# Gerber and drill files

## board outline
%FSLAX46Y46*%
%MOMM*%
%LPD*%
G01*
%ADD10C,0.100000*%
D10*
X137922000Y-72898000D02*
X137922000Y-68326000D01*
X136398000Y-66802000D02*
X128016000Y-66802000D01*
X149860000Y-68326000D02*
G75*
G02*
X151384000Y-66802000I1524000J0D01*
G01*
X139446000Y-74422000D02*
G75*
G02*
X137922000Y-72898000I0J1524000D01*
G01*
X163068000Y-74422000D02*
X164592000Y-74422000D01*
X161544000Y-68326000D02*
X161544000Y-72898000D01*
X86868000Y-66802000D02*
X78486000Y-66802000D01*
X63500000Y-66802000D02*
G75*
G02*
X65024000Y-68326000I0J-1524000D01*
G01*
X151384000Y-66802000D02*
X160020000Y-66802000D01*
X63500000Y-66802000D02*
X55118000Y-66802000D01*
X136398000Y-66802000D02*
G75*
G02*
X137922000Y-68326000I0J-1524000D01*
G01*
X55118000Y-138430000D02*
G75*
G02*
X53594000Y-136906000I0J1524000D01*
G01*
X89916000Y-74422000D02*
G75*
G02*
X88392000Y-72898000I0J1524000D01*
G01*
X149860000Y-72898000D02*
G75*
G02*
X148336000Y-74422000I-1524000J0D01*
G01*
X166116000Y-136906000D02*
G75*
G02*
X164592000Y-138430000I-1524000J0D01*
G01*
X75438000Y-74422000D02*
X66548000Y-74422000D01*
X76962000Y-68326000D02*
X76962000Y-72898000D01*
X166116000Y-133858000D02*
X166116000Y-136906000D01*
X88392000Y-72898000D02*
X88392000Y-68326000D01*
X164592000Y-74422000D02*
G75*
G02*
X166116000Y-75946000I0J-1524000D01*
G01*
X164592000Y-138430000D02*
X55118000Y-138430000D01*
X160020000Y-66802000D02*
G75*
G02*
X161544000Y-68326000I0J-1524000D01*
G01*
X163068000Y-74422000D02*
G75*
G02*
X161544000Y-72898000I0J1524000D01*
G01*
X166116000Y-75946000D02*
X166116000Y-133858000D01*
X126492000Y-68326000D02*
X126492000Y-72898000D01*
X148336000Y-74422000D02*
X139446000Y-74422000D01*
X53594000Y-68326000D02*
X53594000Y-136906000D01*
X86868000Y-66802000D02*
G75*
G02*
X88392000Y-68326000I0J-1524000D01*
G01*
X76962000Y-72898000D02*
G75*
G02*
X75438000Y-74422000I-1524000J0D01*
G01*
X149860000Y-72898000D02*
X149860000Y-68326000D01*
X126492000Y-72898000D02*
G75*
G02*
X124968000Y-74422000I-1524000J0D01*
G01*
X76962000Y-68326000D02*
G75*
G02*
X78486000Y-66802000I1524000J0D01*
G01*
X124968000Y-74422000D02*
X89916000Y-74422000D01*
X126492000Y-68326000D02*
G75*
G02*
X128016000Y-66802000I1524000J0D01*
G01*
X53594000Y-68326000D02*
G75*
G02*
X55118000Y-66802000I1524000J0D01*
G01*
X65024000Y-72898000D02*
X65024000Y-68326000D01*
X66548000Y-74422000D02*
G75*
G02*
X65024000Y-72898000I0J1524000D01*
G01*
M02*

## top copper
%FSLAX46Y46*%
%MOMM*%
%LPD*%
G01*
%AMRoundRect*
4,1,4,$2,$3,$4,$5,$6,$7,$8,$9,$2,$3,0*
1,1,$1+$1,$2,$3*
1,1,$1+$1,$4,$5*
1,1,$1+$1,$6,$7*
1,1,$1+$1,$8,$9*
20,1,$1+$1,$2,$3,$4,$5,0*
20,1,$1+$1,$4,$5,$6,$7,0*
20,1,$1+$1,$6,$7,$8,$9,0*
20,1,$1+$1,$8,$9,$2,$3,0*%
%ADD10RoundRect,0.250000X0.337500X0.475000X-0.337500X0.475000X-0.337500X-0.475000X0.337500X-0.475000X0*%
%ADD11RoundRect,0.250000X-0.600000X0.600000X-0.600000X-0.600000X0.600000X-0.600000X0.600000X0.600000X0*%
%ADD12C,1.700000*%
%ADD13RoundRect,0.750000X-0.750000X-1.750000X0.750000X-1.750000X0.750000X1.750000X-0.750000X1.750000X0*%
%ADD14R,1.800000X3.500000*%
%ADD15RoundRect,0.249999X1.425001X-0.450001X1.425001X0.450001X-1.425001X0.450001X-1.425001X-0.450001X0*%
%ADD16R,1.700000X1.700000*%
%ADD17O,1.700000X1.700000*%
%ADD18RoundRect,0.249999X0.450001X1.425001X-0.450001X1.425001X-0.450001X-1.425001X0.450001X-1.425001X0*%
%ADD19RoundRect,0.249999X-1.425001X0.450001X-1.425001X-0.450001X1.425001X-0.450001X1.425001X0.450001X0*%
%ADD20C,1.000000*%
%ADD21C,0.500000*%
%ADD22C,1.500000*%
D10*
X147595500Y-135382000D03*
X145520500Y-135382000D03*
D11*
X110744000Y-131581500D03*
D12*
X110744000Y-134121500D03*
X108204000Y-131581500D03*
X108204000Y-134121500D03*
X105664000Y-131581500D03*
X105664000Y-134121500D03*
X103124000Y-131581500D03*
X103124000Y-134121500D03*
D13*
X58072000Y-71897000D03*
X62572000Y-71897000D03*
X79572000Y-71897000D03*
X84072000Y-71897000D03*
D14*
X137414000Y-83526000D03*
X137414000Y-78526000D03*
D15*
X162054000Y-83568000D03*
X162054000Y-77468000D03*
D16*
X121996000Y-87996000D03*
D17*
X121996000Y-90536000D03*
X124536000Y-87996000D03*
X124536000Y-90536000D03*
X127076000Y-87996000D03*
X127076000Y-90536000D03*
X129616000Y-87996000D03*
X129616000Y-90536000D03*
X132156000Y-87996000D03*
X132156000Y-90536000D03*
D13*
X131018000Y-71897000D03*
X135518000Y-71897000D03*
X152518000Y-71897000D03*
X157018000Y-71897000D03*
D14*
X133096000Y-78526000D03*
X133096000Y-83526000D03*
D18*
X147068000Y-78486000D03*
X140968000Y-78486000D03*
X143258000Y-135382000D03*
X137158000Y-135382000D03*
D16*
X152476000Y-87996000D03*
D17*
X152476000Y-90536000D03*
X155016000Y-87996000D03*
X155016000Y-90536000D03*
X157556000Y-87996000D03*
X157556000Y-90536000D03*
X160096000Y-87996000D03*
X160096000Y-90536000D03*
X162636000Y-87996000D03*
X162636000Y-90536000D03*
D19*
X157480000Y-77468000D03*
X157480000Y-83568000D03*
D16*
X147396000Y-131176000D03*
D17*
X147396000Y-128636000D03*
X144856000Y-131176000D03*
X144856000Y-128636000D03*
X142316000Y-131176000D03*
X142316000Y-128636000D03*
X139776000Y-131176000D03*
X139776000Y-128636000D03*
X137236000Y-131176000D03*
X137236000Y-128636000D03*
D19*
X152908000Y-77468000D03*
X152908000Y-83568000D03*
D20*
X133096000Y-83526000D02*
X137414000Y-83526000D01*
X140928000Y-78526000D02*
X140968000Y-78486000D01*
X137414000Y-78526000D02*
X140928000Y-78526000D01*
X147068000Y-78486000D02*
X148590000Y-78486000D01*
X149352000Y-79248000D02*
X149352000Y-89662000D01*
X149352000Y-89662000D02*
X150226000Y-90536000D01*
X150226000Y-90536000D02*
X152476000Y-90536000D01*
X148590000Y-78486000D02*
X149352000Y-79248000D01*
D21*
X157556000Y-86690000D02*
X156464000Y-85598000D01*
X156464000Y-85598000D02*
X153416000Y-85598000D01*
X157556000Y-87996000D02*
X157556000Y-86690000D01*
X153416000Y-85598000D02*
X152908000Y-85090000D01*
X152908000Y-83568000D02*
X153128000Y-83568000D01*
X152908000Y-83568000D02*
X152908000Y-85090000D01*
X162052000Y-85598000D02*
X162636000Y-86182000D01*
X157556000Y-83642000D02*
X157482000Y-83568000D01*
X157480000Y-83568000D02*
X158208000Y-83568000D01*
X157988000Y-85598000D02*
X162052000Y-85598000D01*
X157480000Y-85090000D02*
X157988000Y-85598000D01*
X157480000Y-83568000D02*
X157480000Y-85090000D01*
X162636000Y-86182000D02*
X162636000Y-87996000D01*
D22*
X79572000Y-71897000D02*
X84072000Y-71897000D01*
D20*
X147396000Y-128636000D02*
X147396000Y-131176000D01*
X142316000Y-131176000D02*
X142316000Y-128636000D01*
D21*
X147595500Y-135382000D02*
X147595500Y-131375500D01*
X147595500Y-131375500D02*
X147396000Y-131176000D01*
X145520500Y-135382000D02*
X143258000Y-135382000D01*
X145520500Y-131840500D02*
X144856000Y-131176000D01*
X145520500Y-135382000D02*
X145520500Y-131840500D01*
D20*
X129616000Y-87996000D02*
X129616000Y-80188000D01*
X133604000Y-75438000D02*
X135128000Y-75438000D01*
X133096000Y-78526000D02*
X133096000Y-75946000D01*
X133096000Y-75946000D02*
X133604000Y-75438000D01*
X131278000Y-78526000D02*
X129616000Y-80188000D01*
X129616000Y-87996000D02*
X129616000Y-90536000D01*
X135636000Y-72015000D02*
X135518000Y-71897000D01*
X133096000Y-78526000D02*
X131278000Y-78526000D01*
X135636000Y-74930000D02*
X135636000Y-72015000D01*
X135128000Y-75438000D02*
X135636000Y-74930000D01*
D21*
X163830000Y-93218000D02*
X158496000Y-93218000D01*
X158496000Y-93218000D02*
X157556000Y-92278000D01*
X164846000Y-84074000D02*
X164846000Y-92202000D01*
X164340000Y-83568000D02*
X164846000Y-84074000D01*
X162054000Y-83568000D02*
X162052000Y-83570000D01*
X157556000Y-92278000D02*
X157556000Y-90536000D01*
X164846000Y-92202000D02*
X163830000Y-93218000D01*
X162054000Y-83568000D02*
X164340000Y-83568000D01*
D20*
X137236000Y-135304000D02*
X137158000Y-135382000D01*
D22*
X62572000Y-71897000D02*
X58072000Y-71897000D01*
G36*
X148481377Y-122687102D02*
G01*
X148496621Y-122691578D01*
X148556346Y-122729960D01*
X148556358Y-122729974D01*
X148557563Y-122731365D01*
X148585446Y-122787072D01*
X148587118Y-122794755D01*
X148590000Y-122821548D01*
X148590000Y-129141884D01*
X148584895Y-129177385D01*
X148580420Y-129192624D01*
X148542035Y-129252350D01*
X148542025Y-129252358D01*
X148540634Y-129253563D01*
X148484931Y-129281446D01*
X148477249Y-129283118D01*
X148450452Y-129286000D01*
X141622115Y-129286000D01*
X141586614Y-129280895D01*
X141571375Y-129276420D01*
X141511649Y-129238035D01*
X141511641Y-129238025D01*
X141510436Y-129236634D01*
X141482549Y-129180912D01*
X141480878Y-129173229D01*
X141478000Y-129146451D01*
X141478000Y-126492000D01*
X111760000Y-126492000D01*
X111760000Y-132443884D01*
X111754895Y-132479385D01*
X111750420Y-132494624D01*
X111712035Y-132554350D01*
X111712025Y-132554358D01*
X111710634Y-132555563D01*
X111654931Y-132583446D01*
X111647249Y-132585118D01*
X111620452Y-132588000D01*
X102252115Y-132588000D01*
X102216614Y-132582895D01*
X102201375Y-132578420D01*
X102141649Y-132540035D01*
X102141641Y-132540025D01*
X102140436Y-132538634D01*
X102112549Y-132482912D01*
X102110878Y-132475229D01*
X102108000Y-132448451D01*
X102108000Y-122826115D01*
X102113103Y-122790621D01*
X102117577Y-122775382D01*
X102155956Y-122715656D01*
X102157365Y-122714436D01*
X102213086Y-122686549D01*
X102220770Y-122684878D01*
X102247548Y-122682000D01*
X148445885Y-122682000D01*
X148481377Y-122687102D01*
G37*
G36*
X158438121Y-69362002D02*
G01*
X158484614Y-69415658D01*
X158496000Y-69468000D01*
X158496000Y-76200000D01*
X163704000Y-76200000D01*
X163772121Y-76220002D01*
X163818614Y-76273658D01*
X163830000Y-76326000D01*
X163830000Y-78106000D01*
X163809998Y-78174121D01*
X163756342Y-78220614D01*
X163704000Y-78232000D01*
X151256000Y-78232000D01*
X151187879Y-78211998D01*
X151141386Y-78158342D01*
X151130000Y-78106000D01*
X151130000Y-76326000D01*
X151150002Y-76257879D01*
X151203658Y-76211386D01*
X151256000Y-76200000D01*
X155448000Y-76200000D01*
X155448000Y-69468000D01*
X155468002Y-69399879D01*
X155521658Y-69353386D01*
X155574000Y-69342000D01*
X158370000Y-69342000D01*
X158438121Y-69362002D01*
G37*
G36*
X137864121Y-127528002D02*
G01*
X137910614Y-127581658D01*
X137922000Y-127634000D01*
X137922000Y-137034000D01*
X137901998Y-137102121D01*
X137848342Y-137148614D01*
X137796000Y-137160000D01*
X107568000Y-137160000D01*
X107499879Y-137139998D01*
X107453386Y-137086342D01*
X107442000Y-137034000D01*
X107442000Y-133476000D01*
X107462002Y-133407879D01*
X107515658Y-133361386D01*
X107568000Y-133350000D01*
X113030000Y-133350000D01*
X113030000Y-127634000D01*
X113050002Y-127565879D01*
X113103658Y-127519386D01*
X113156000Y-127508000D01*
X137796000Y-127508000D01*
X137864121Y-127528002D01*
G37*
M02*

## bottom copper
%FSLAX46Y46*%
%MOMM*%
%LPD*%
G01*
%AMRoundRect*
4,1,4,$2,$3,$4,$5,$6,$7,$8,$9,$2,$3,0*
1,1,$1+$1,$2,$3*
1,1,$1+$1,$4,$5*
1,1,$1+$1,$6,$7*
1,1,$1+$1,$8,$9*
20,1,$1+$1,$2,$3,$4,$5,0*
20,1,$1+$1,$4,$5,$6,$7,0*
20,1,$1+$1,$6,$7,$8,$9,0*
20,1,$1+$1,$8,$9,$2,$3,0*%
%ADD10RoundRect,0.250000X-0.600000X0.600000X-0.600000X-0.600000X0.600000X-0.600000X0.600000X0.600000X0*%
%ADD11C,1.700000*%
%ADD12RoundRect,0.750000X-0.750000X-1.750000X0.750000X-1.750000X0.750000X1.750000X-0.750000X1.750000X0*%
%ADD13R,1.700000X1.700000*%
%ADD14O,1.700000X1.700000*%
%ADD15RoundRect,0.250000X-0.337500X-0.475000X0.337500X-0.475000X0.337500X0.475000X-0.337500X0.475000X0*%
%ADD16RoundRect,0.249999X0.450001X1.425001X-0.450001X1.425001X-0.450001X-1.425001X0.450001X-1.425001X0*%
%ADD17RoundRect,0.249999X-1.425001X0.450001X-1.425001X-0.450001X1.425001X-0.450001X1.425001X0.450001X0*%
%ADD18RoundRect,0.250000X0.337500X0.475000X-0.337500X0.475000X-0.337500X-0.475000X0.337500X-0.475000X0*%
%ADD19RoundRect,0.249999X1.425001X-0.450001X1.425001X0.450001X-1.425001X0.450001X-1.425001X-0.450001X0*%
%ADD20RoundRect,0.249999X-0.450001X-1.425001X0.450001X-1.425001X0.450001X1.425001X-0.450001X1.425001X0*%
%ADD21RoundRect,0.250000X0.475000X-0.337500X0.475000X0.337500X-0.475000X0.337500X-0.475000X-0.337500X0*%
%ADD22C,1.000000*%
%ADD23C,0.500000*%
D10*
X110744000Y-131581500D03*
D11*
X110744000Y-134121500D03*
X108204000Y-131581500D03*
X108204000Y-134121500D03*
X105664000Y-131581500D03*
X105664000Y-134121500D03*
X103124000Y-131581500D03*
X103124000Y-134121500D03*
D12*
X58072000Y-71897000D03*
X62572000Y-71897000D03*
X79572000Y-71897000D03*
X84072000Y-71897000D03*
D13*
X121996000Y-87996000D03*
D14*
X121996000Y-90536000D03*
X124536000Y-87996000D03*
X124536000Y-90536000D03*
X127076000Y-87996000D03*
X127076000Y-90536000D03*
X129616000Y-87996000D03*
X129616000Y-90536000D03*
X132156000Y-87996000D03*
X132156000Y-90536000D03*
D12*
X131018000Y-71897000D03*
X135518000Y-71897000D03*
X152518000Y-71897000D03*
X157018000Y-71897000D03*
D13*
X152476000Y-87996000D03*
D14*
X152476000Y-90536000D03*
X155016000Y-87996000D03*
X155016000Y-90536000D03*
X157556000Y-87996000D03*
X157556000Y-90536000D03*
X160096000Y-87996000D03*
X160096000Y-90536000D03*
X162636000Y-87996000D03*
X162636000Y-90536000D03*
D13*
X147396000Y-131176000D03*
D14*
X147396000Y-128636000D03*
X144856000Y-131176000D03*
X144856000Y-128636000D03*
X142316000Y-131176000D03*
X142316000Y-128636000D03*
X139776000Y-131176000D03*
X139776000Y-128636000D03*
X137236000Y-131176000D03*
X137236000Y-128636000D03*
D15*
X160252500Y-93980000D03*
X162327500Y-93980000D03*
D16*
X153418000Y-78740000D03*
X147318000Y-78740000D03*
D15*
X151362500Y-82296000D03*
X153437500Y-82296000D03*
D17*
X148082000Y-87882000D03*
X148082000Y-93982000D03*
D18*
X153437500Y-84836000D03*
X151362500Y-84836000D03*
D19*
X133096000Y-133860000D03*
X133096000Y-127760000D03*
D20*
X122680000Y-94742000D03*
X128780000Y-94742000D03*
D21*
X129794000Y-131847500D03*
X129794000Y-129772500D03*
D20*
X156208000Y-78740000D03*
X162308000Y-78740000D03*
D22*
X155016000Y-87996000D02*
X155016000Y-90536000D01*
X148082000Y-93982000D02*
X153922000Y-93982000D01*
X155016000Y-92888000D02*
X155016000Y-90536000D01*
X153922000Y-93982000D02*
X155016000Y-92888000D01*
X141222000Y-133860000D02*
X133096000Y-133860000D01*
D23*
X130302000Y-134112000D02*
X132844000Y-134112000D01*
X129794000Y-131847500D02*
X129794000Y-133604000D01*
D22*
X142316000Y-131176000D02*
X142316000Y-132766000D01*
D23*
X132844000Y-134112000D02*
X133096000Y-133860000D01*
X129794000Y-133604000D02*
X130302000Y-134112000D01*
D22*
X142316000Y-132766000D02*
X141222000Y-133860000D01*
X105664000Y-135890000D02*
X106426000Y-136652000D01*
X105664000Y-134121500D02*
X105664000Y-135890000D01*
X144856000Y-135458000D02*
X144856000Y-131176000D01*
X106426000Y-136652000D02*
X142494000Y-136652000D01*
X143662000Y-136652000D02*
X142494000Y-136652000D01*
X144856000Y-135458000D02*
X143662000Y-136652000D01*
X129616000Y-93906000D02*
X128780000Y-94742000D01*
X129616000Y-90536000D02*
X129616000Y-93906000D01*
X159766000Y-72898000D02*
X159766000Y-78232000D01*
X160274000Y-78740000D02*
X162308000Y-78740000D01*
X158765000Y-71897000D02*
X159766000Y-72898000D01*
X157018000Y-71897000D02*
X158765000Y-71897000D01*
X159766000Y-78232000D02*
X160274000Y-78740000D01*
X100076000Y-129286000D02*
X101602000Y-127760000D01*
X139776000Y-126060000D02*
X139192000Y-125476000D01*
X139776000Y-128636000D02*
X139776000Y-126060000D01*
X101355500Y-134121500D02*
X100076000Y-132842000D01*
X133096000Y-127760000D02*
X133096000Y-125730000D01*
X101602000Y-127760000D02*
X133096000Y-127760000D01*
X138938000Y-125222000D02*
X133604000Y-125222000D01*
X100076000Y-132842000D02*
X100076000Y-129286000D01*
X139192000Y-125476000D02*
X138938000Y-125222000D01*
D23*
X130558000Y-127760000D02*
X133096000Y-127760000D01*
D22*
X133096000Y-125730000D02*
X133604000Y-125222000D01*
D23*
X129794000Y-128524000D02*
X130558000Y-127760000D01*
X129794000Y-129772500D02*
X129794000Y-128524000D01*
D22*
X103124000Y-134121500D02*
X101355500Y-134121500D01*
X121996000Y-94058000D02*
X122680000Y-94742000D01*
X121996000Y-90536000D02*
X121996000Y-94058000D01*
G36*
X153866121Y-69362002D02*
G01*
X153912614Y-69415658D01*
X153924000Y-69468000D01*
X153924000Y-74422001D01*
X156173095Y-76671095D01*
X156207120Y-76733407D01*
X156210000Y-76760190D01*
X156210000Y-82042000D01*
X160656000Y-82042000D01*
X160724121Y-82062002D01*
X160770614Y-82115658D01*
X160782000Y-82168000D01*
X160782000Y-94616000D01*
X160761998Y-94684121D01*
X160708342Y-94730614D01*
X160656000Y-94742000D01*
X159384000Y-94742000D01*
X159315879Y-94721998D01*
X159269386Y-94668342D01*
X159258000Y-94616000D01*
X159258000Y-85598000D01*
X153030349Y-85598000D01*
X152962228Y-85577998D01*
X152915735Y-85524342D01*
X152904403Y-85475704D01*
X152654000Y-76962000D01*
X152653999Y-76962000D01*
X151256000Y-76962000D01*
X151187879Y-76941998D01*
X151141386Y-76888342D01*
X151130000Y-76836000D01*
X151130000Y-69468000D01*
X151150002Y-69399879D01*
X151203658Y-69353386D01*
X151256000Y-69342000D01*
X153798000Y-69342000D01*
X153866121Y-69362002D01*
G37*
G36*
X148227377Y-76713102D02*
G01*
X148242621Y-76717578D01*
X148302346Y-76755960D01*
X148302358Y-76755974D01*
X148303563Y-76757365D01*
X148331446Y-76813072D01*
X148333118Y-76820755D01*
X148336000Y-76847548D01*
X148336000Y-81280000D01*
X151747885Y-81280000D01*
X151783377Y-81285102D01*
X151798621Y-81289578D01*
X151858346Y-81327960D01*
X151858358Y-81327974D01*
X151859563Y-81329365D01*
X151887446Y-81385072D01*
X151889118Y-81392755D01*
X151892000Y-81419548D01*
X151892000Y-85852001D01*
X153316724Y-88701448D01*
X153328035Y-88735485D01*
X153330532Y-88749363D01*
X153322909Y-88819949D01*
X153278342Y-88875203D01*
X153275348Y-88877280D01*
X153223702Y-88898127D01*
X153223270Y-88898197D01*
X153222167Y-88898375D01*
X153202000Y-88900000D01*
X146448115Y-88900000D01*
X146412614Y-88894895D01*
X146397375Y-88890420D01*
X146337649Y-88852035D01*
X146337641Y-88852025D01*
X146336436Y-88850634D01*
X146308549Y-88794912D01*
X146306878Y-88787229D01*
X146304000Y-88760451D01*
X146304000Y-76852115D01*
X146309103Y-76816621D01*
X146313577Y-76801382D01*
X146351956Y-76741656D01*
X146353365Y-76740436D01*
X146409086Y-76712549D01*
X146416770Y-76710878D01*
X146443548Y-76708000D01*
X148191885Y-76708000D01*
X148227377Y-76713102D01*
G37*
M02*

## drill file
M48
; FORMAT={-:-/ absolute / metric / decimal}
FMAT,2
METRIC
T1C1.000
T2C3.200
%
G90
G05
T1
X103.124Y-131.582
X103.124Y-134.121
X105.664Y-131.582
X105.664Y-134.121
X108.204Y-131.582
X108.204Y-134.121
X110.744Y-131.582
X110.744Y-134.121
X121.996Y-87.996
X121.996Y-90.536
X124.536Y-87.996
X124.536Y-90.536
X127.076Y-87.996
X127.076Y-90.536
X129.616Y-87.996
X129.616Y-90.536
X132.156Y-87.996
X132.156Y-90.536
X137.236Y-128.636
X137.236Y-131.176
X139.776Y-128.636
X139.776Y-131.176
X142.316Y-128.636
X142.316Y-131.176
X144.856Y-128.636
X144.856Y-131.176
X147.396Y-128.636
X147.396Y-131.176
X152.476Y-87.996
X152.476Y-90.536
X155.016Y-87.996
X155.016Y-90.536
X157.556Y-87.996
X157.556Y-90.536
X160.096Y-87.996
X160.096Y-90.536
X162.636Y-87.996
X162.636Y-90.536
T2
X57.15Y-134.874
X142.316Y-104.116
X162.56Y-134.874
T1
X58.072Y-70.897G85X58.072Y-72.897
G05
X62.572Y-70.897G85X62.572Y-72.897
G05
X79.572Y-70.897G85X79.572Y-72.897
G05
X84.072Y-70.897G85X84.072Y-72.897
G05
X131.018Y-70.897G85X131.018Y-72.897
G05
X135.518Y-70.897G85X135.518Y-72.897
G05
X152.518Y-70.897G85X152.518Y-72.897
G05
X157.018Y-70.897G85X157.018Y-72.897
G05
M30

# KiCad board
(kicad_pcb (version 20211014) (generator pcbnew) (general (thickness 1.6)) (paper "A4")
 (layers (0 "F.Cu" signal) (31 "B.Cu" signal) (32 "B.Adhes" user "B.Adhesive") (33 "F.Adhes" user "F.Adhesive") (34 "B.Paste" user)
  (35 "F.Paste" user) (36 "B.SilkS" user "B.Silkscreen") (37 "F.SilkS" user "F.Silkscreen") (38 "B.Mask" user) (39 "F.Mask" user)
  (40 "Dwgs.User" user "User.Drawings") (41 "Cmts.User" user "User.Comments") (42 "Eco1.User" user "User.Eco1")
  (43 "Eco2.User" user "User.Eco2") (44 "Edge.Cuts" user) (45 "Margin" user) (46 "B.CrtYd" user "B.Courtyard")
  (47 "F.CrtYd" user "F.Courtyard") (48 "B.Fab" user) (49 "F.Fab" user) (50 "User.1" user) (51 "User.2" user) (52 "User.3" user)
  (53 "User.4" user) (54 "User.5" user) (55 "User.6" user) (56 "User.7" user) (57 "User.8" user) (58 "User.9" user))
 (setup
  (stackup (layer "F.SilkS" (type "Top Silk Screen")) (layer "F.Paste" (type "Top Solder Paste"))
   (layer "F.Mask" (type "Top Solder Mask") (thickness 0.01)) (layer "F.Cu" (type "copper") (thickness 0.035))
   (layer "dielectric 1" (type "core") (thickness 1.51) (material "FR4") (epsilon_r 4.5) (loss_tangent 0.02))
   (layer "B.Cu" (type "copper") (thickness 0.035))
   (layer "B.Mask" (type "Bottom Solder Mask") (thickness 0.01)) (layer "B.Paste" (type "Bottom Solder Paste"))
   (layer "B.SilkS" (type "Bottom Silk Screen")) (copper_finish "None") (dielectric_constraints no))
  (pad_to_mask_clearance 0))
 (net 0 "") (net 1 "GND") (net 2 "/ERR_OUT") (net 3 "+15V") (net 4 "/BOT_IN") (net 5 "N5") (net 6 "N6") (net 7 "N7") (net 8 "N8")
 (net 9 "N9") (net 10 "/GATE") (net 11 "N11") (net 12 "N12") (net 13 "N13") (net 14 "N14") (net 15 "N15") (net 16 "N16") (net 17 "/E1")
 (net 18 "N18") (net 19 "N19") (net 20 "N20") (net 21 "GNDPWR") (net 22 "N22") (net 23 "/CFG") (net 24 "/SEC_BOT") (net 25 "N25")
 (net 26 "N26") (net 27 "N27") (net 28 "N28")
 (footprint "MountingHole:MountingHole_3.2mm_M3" (layer "F.Cu") (at 57.15 134.874)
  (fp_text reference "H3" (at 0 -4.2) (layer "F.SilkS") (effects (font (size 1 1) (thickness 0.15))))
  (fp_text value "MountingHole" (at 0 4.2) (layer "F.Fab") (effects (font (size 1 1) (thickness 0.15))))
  (pad "" np_thru_hole circle (at 0 0) (size 3.2 3.2) (drill 3.2) (layers *.Cu *.Mask)))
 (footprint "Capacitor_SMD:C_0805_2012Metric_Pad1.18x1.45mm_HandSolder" (layer "F.Cu") (at 146.558 135.382 180)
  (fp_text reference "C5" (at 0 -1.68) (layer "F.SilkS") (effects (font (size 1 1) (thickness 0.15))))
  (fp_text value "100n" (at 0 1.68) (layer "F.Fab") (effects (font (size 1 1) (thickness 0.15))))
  (pad "1" smd roundrect (at -1.0375 0 180) (size 1.175 1.45) (layers "F.Cu" "F.Paste" "F.Mask") (roundrect_rratio 0.212766) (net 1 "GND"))
  (pad "2" smd roundrect (at 1.0375 0 180) (size 1.175 1.45) (layers "F.Cu" "F.Paste" "F.Mask") (roundrect_rratio 0.212766)
   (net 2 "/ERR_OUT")))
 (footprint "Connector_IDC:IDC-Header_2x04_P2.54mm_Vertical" (layer "F.Cu") (at 110.744 131.5815 -90)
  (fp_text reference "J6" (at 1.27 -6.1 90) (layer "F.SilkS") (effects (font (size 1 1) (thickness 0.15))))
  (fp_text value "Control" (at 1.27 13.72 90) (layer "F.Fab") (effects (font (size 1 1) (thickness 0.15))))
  (pad "1" thru_hole roundrect (at 0 0 270) (size 1.7 1.7) (drill 1) (layers *.Cu *.Mask) (roundrect_rratio 0.147059) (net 1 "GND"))
  (pad "2" thru_hole circle (at 2.54 0 270) (size 1.7 1.7) (drill 1) (layers *.Cu *.Mask) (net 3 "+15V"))
  (pad "3" thru_hole circle (at 0 2.54 270) (size 1.7 1.7) (drill 1) (layers *.Cu *.Mask) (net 1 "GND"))
  (pad "4" thru_hole circle (at 2.54 2.54 270) (size 1.7 1.7) (drill 1) (layers *.Cu *.Mask) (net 3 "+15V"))
  (pad "5" thru_hole circle (at 0 5.08 270) (size 1.7 1.7) (drill 1) (layers *.Cu *.Mask) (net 1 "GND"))
  (pad "6" thru_hole circle (at 2.54 5.08 270) (size 1.7 1.7) (drill 1) (layers *.Cu *.Mask) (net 2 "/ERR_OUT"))
  (pad "7" thru_hole circle (at 0 7.62 270) (size 1.7 1.7) (drill 1) (layers *.Cu *.Mask) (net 1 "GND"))
  (pad "8" thru_hole circle (at 2.54 7.62 270) (size 1.7 1.7) (drill 1) (layers *.Cu *.Mask) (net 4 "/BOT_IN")))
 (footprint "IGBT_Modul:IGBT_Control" (layer "F.Cu") (at 71.072 61.897)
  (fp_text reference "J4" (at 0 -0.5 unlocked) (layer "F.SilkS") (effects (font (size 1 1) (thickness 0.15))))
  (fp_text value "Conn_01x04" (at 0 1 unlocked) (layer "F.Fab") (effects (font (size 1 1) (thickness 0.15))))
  (pad "1" thru_hole roundrect (at -13 10) (size 3 5) (drill oval 1 3) (layers *.Cu *.Mask) (roundrect_rratio 0.25) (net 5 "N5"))
  (pad "2" thru_hole roundrect (at -8.5 10) (size 3 5) (drill oval 1 3) (layers *.Cu *.Mask) (roundrect_rratio 0.25) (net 5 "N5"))
  (pad "3" thru_hole roundrect (at 8.5 10) (size 3 5) (drill oval 1 3) (layers *.Cu *.Mask) (roundrect_rratio 0.25) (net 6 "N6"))
  (pad "4" thru_hole roundrect (at 13 10) (size 3 5) (drill oval 1 3) (layers *.Cu *.Mask) (roundrect_rratio 0.25) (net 6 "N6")))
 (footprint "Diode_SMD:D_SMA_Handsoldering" (layer "F.Cu") (at 137.414 81.026 90)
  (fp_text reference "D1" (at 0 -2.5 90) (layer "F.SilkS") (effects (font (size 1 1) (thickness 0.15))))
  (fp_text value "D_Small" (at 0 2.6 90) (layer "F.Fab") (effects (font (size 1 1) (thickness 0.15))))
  (pad "1" smd rect (at -2.5 0 90) (size 3.5 1.8) (layers "F.Cu" "F.Paste" "F.Mask") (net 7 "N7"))
  (pad "2" smd rect (at 2.5 0 90) (size 3.5 1.8) (layers "F.Cu" "F.Paste" "F.Mask") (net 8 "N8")))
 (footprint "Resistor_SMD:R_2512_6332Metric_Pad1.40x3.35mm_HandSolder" (layer "F.Cu") (at 162.054 80.518 90)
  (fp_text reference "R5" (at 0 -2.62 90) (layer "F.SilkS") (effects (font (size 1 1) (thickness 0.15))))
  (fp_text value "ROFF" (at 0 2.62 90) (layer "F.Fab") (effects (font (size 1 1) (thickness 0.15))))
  (pad "1" smd roundrect (at -3.05 0 90) (size 1.4 3.35) (layers "F.Cu" "F.Paste" "F.Mask") (roundrect_rratio 0.178571) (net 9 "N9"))
  (pad "2" smd roundrect (at 3.05 0 90) (size 1.4 3.35) (layers "F.Cu" "F.Paste" "F.Mask") (roundrect_rratio 0.178571) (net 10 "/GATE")))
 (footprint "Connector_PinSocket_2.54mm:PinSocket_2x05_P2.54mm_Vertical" (layer "F.Cu") (at 121.996 87.996 90)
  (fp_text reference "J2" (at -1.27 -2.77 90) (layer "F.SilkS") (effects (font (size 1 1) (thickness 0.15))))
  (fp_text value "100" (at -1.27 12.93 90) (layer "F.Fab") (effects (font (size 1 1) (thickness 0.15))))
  (pad "1" thru_hole rect (at 0 0 90) (size 1.7 1.7) (drill 1) (layers *.Cu *.Mask) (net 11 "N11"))
  (pad "2" thru_hole oval (at -2.54 0 90) (size 1.7 1.7) (drill 1) (layers *.Cu *.Mask) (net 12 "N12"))
  (pad "3" thru_hole oval (at 0 2.54 90) (size 1.7 1.7) (drill 1) (layers *.Cu *.Mask) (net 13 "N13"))
  (pad "4" thru_hole oval (at -2.54 2.54 90) (size 1.7 1.7) (drill 1) (layers *.Cu *.Mask) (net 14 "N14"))
  (pad "5" thru_hole oval (at 0 5.08 90) (size 1.7 1.7) (drill 1) (layers *.Cu *.Mask) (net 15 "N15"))
  (pad "6" thru_hole oval (at -2.54 5.08 90) (size 1.7 1.7) (drill 1) (layers *.Cu *.Mask) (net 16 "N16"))
  (pad "7" thru_hole oval (at 0 7.62 90) (size 1.7 1.7) (drill 1) (layers *.Cu *.Mask) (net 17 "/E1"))
  (pad "8" thru_hole oval (at -2.54 7.62 90) (size 1.7 1.7) (drill 1) (layers *.Cu *.Mask) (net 17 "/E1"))
  (pad "9" thru_hole oval (at 0 10.16 90) (size 1.7 1.7) (drill 1) (layers *.Cu *.Mask) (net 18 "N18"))
  (pad "10" thru_hole oval (at -2.54 10.16 90) (size 1.7 1.7) (drill 1) (layers *.Cu *.Mask) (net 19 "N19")))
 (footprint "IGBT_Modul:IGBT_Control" (layer "F.Cu") (at 144.018 61.897)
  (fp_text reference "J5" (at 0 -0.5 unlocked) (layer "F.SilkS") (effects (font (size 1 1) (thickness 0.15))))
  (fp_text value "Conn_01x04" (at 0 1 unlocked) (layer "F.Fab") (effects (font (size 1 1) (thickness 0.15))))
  (pad "1" thru_hole roundrect (at -13 10) (size 3 5) (drill oval 1 3) (layers *.Cu *.Mask) (roundrect_rratio 0.25) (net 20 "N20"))
  (pad "2" thru_hole roundrect (at -8.5 10) (size 3 5) (drill oval 1 3) (layers *.Cu *.Mask) (roundrect_rratio 0.25) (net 17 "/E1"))
  (pad "3" thru_hole roundrect (at 8.5 10) (size 3 5) (drill oval 1 3) (layers *.Cu *.Mask) (roundrect_rratio 0.25) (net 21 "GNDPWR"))
  (pad "4" thru_hole roundrect (at 13 10) (size 3 5) (drill oval 1 3) (layers *.Cu *.Mask) (roundrect_rratio 0.25) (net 10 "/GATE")))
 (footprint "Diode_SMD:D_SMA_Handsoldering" (layer "F.Cu") (at 133.096 81.026 -90)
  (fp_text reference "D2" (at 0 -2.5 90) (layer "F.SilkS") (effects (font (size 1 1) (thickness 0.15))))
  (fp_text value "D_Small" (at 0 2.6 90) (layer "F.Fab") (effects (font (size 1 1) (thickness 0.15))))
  (pad "1" smd rect (at -2.5 0 270) (size 3.5 1.8) (layers "F.Cu" "F.Paste" "F.Mask") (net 17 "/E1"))
  (pad "2" smd rect (at 2.5 0 270) (size 3.5 1.8) (layers "F.Cu" "F.Paste" "F.Mask") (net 7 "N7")))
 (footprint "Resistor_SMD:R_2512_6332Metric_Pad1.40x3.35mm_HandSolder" (layer "F.Cu") (at 144.018 78.486 180)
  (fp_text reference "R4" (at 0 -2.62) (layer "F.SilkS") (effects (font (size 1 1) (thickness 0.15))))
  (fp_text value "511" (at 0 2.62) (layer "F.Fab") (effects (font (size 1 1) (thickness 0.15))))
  (pad "1" smd roundrect (at -3.05 0 180) (size 1.4 3.35) (layers "F.Cu" "F.Paste" "F.Mask") (roundrect_rratio 0.178571) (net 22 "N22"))
  (pad "2" smd roundrect (at 3.05 0 180) (size 1.4 3.35) (layers "F.Cu" "F.Paste" "F.Mask") (roundrect_rratio 0.178571) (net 8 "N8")))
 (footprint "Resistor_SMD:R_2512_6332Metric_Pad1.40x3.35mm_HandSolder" (layer "F.Cu") (at 140.208 135.382 180)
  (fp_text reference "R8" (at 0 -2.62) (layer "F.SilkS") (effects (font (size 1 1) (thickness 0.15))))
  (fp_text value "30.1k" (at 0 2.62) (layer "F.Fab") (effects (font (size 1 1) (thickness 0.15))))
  (pad "1" smd roundrect (at -3.05 0 180) (size 1.4 3.35) (layers "F.Cu" "F.Paste" "F.Mask") (roundrect_rratio 0.178571) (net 2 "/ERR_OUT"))
  (pad "2" smd roundrect (at 3.05 0 180) (size 1.4 3.35) (layers "F.Cu" "F.Paste" "F.Mask") (roundrect_rratio 0.178571) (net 3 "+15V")))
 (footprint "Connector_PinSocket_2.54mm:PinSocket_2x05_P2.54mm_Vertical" (layer "F.Cu") (at 152.476 87.996 90)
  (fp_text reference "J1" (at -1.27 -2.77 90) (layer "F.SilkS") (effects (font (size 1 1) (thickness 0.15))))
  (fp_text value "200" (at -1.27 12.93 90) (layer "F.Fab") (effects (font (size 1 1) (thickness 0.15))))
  (pad "1" thru_hole rect (at 0 0 90) (size 1.7 1.7) (drill 1) (layers *.Cu *.Mask) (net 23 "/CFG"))
  (pad "2" thru_hole oval (at -2.54 0 90) (size 1.7 1.7) (drill 1) (layers *.Cu *.Mask) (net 22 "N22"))
  (pad "3" thru_hole oval (at 0 2.54 90) (size 1.7 1.7) (drill 1) (layers *.Cu *.Mask) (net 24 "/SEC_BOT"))
  (pad "4" thru_hole oval (at -2.54 2.54 90) (size 1.7 1.7) (drill 1) (layers *.Cu *.Mask) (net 24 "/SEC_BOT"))
  (pad "5" thru_hole oval (at 0 5.08 90) (size 1.7 1.7) (drill 1) (layers *.Cu *.Mask) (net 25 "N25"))
  (pad "6" thru_hole oval (at -2.54 5.08 90) (size 1.7 1.7) (drill 1) (layers *.Cu *.Mask) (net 9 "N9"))
  (pad "7" thru_hole oval (at 0 7.62 90) (size 1.7 1.7) (drill 1) (layers *.Cu *.Mask) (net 21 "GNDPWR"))
  (pad "8" thru_hole oval (at -2.54 7.62 90) (size 1.7 1.7) (drill 1) (layers *.Cu *.Mask) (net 21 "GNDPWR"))
  (pad "9" thru_hole oval (at 0 10.16 90) (size 1.7 1.7) (drill 1) (layers *.Cu *.Mask) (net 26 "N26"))
  (pad "10" thru_hole oval (at -2.54 10.16 90) (size 1.7 1.7) (drill 1) (layers *.Cu *.Mask) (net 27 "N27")))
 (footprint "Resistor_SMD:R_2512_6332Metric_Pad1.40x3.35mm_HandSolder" (layer "F.Cu") (at 157.48 80.518 -90)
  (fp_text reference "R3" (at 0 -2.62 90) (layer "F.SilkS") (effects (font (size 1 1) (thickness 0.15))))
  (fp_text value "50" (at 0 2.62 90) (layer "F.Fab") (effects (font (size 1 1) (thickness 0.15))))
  (pad "1" smd roundrect (at -3.05 0 270) (size 1.4 3.35) (layers "F.Cu" "F.Paste" "F.Mask") (roundrect_rratio 0.178571) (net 10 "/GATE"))
  (pad "2" smd roundrect (at 3.05 0 270) (size 1.4 3.35) (layers "F.Cu" "F.Paste" "F.Mask") (roundrect_rratio 0.178571) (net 26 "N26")))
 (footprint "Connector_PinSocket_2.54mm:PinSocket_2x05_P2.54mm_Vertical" (layer "F.Cu") (at 147.396 131.176 -90)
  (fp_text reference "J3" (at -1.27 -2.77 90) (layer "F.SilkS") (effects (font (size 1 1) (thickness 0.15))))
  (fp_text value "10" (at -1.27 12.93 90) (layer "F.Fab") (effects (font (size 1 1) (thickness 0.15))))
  (pad "1" thru_hole rect (at 0 0 270) (size 1.7 1.7) (drill 1) (layers *.Cu *.Mask) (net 1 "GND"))
  (pad "2" thru_hole oval (at -2.54 0 270) (size 1.7 1.7) (drill 1) (layers *.Cu *.Mask) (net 1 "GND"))
  (pad "3" thru_hole oval (at 0 2.54 270) (size 1.7 1.7) (drill 1) (layers *.Cu *.Mask) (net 2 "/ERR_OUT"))
  (pad "4" thru_hole oval (at -2.54 2.54 270) (size 1.7 1.7) (drill 1) (layers *.Cu *.Mask) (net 1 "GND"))
  (pad "5" thru_hole oval (at 0 5.08 270) (size 1.7 1.7) (drill 1) (layers *.Cu *.Mask) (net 1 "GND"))
  (pad "6" thru_hole oval (at -2.54 5.08 270) (size 1.7 1.7) (drill 1) (layers *.Cu *.Mask) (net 1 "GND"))
  (pad "7" thru_hole oval (at 0 7.62 270) (size 1.7 1.7) (drill 1) (layers *.Cu *.Mask) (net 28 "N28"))
  (pad "8" thru_hole oval (at -2.54 7.62 270) (size 1.7 1.7) (drill 1) (layers *.Cu *.Mask) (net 4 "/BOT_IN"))
  (pad "9" thru_hole oval (at 0 10.16 270) (size 1.7 1.7) (drill 1) (layers *.Cu *.Mask) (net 3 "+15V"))
  (pad "10" thru_hole oval (at -2.54 10.16 270) (size 1.7 1.7) (drill 1) (layers *.Cu *.Mask) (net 3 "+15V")))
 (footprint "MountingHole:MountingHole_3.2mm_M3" (layer "F.Cu") (at 142.316 104.116)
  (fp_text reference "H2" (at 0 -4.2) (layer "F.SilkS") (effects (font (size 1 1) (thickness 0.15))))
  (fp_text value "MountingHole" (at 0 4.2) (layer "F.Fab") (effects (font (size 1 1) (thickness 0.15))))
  (pad "" np_thru_hole circle (at 0 0) (size 3.2 3.2) (drill 3.2) (layers *.Cu *.Mask)))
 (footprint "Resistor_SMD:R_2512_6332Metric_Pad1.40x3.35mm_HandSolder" (layer "F.Cu") (at 152.908 80.518 -90)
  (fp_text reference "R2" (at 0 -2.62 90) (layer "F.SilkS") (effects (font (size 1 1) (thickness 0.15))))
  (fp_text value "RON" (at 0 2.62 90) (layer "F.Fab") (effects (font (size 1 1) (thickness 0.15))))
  (pad "1" smd roundrect (at -3.05 0 270) (size 1.4 3.35) (layers "F.Cu" "F.Paste" "F.Mask") (roundrect_rratio 0.178571) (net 10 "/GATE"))
  (pad "2" smd roundrect (at 3.05 0 270) (size 1.4 3.35) (layers "F.Cu" "F.Paste" "F.Mask") (roundrect_rratio 0.178571) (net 25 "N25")))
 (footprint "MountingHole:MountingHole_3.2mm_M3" (layer "F.Cu") (at 162.56 134.874)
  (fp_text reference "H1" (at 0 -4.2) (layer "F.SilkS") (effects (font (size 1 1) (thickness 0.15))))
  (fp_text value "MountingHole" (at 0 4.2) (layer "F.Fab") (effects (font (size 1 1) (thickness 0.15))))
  (pad "" np_thru_hole circle (at 0 0) (size 3.2 3.2) (drill 3.2) (layers *.Cu *.Mask)))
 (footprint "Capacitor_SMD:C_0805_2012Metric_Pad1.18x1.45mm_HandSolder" (layer "B.Cu") (at 161.29 93.98)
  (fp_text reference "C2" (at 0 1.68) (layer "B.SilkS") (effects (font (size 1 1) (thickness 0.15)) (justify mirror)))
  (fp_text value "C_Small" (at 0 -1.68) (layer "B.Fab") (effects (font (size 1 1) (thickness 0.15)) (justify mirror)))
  (pad "1" smd roundrect (at -1.0375 0) (size 1.175 1.45) (layers "B.Cu" "B.Paste" "B.Mask") (roundrect_rratio 0.212766) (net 21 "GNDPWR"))
  (pad "2" smd roundrect (at 1.0375 0) (size 1.175 1.45) (layers "B.Cu" "B.Paste" "B.Mask") (roundrect_rratio 0.212766) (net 27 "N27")))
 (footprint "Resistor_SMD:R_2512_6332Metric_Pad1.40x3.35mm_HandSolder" (layer "B.Cu") (at 150.368 78.74 180)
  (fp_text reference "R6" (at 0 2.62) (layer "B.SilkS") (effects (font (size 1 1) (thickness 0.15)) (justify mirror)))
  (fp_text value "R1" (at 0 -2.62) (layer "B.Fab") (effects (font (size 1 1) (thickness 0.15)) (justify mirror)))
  (pad "1" smd roundrect (at -3.05 0 180) (size 1.4 3.35) (layers "B.Cu" "B.Paste" "B.Mask") (roundrect_rratio 0.178571) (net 21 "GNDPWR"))
  (pad "2" smd roundrect (at 3.05 0 180) (size 1.4 3.35) (layers "B.Cu" "B.Paste" "B.Mask") (roundrect_rratio 0.178571) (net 23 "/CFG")))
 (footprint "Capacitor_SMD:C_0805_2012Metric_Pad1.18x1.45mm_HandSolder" (layer "B.Cu") (at 152.4 82.296)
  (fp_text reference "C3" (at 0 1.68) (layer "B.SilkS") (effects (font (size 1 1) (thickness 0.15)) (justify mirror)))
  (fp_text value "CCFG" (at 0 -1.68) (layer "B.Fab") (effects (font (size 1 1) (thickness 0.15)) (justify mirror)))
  (pad "1" smd roundrect (at -1.0375 0) (size 1.175 1.45) (layers "B.Cu" "B.Paste" "B.Mask") (roundrect_rratio 0.212766) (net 23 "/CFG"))
  (pad "2" smd roundrect (at 1.0375 0) (size 1.175 1.45) (layers "B.Cu" "B.Paste" "B.Mask") (roundrect_rratio 0.212766) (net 21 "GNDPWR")))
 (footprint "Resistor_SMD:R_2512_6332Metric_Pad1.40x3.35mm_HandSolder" (layer "B.Cu") (at 148.082 90.932 -90)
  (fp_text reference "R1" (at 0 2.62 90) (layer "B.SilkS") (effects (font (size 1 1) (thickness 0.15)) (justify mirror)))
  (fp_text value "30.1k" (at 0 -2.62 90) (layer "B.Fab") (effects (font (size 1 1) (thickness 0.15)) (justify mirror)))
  (pad "1" smd roundrect (at -3.05 0 270) (size 1.4 3.35) (layers "B.Cu" "B.Paste" "B.Mask") (roundrect_rratio 0.178571) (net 23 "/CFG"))
  (pad "2" smd roundrect (at 3.05 0 270) (size 1.4 3.35) (layers "B.Cu" "B.Paste" "B.Mask") (roundrect_rratio 0.178571) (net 24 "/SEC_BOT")))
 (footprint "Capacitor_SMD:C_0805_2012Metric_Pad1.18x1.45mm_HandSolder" (layer "B.Cu") (at 152.4 84.836 180)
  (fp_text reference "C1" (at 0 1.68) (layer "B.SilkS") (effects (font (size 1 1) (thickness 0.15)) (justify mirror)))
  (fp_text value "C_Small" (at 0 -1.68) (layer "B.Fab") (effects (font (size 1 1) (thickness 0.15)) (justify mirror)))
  (pad "1" smd roundrect (at -1.0375 0 180) (size 1.175 1.45) (layers "B.Cu" "B.Paste" "B.Mask") (roundrect_rratio 0.212766)
   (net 21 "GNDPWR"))
  (pad "2" smd roundrect (at 1.0375 0 180) (size 1.175 1.45) (layers "B.Cu" "B.Paste" "B.Mask") (roundrect_rratio 0.212766) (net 23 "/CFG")))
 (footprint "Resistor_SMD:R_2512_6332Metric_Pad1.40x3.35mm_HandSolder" (layer "B.Cu") (at 133.096 130.81 90)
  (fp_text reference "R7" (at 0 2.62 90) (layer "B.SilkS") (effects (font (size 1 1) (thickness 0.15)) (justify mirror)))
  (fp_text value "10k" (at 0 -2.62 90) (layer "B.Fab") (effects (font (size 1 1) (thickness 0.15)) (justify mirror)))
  (pad "1" smd roundrect (at -3.05 0 90) (size 1.4 3.35) (layers "B.Cu" "B.Paste" "B.Mask") (roundrect_rratio 0.178571) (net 1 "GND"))
  (pad "2" smd roundrect (at 3.05 0 90) (size 1.4 3.35) (layers "B.Cu" "B.Paste" "B.Mask") (roundrect_rratio 0.178571) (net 4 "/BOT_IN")))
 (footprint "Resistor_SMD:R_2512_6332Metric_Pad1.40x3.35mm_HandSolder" (layer "B.Cu") (at 125.73 94.742)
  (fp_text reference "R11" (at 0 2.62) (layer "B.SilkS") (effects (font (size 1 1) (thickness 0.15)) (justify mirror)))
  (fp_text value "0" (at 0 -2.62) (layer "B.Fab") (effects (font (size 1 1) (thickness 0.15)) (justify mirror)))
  (pad "1" smd roundrect (at -3.05 0) (size 1.4 3.35) (layers "B.Cu" "B.Paste" "B.Mask") (roundrect_rratio 0.178571) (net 12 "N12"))
  (pad "2" smd roundrect (at 3.05 0) (size 1.4 3.35) (layers "B.Cu" "B.Paste" "B.Mask") (roundrect_rratio 0.178571) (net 17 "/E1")))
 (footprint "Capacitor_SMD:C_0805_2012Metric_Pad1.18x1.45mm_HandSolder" (layer "B.Cu") (at 129.794 130.81 90)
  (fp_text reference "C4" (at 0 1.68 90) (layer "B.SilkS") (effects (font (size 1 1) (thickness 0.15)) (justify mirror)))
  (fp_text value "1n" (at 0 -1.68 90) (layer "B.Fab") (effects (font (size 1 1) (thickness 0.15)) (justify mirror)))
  (pad "1" smd roundrect (at -1.0375 0 90) (size 1.175 1.45) (layers "B.Cu" "B.Paste" "B.Mask") (roundrect_rratio 0.212766) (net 1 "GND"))
  (pad "2" smd roundrect (at 1.0375 0 90) (size 1.175 1.45) (layers "B.Cu" "B.Paste" "B.Mask") (roundrect_rratio 0.212766) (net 4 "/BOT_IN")))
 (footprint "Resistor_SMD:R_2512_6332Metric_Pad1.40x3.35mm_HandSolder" (layer "B.Cu") (at 159.258 78.74)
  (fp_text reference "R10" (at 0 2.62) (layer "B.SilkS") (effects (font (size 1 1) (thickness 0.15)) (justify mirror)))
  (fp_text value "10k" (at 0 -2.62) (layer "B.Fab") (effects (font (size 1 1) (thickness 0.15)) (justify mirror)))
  (pad "1" smd roundrect (at -3.05 0) (size 1.4 3.35) (layers "B.Cu" "B.Paste" "B.Mask") (roundrect_rratio 0.178571) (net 21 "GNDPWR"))
  (pad "2" smd roundrect (at 3.05 0) (size 1.4 3.35) (layers "B.Cu" "B.Paste" "B.Mask") (roundrect_rratio 0.178571) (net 10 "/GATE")))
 (gr_line (start 137.922 72.898) (end 137.922 68.326) (layer "Edge.Cuts") (width 0.1))
 (gr_line (start 136.398 66.802) (end 128.016 66.802) (layer "Edge.Cuts") (width 0.1))
 (gr_arc (start 149.86 68.326) (mid 150.306369 67.248369) (end 151.384 66.802) (layer "Edge.Cuts") (width 0.1))
 (gr_arc (start 139.446 74.422) (mid 138.368369 73.975631) (end 137.922 72.898) (layer "Edge.Cuts") (width 0.1))
 (gr_line (start 163.068 74.422) (end 164.592 74.422) (layer "Edge.Cuts") (width 0.1))
 (gr_line (start 161.544 68.326) (end 161.544 72.898) (layer "Edge.Cuts") (width 0.1))
 (gr_line (start 86.868 66.802) (end 78.486 66.802) (layer "Edge.Cuts") (width 0.1))
 (gr_arc (start 63.5 66.802) (mid 64.577631 67.248369) (end 65.024 68.326) (layer "Edge.Cuts") (width 0.1))
 (gr_line (start 151.384 66.802) (end 160.02 66.802) (layer "Edge.Cuts") (width 0.1))
 (gr_line (start 63.5 66.802) (end 55.118 66.802) (layer "Edge.Cuts") (width 0.1))
 (gr_arc (start 136.398 66.802) (mid 137.475631 67.248369) (end 137.922 68.326) (layer "Edge.Cuts") (width 0.1))
 (gr_arc (start 55.118 138.43) (mid 54.040369 137.983631) (end 53.594 136.906) (layer "Edge.Cuts") (width 0.1))
 (gr_arc (start 89.916 74.422) (mid 88.838369 73.975631) (end 88.392 72.898) (layer "Edge.Cuts") (width 0.1))
 (gr_arc (start 149.86 72.898) (mid 149.413631 73.975631) (end 148.336 74.422) (layer "Edge.Cuts") (width 0.1))
 (gr_arc (start 166.116 136.906) (mid 165.669631 137.983631) (end 164.592 138.43) (layer "Edge.Cuts") (width 0.1))
 (gr_line (start 75.438 74.422) (end 66.548 74.422) (layer "Edge.Cuts") (width 0.1))
 (gr_line (start 76.962 68.326) (end 76.962 72.898) (layer "Edge.Cuts") (width 0.1))
 (gr_line (start 166.116 133.858) (end 166.116 136.906) (layer "Edge.Cuts") (width 0.1))
 (gr_line (start 88.392 72.898) (end 88.392 68.326) (layer "Edge.Cuts") (width 0.1))
 (gr_arc (start 164.592 74.422) (mid 165.669631 74.868369) (end 166.116 75.946) (layer "Edge.Cuts") (width 0.1))
 (gr_line (start 164.592 138.43) (end 55.118 138.43) (layer "Edge.Cuts") (width 0.1))
 (gr_arc (start 160.02 66.802) (mid 161.097631 67.248369) (end 161.544 68.326) (layer "Edge.Cuts") (width 0.1))
 (gr_arc (start 163.068 74.422) (mid 161.990369 73.975631) (end 161.544 72.898) (layer "Edge.Cuts") (width 0.1))
 (gr_line (start 166.116 75.946) (end 166.116 133.858) (layer "Edge.Cuts") (width 0.1))
 (gr_line (start 126.492 68.326) (end 126.492 72.898) (layer "Edge.Cuts") (width 0.1))
 (gr_line (start 148.336 74.422) (end 139.446 74.422) (layer "Edge.Cuts") (width 0.1))
 (gr_line (start 53.594 68.326) (end 53.594 136.906) (layer "Edge.Cuts") (width 0.1))
 (gr_arc (start 86.868 66.802) (mid 87.945631 67.248369) (end 88.392 68.326) (layer "Edge.Cuts") (width 0.1))
 (gr_arc (start 76.962 72.898) (mid 76.515631 73.975631) (end 75.438 74.422) (layer "Edge.Cuts") (width 0.1))
 (gr_line (start 149.86 72.898) (end 149.86 68.326) (layer "Edge.Cuts") (width 0.1))
 (gr_arc (start 126.492 72.898) (mid 126.045631 73.975631) (end 124.968 74.422) (layer "Edge.Cuts") (width 0.1))
 (gr_arc (start 76.962 68.326) (mid 77.408369 67.248369) (end 78.486 66.802) (layer "Edge.Cuts") (width 0.1))
 (gr_line (start 124.968 74.422) (end 89.916 74.422) (layer "Edge.Cuts") (width 0.1))
 (gr_arc (start 126.492 68.326) (mid 126.938369 67.248369) (end 128.016 66.802) (layer "Edge.Cuts") (width 0.1))
 (gr_arc (start 53.594 68.326) (mid 54.040369 67.248369) (end 55.118 66.802) (layer "Edge.Cuts") (width 0.1))
 (gr_line (start 65.024 72.898) (end 65.024 68.326) (layer "Edge.Cuts") (width 0.1))
 (gr_arc (start 66.548 74.422) (mid 65.470369 73.975631) (end 65.024 72.898) (layer "Edge.Cuts") (width 0.1))
 (segment (start 155.016 87.996) (end 155.016 90.536) (width 1) (layer "B.Cu") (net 24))
 (segment (start 148.082 93.982) (end 153.922 93.982) (width 1) (layer "B.Cu") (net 24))
 (segment (start 155.016 92.888) (end 155.016 90.536) (width 1) (layer "B.Cu") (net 24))
 (segment (start 153.922 93.982) (end 155.016 92.888) (width 1) (layer "B.Cu") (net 24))
 (segment (start 133.096 83.526) (end 137.414 83.526) (width 1) (layer "F.Cu") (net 7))
 (segment (start 140.928 78.526) (end 140.968 78.486) (width 1) (layer "F.Cu") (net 8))
 (segment (start 137.414 78.526) (end 140.928 78.526) (width 1) (layer "F.Cu") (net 8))
 (segment (start 147.068 78.486) (end 148.59 78.486) (width 1) (layer "F.Cu") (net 22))
 (segment (start 149.352 79.248) (end 149.352 89.662) (width 1) (layer "F.Cu") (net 22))
 (segment (start 149.352 89.662) (end 150.226 90.536) (width 1) (layer "F.Cu") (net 22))
 (segment (start 150.226 90.536) (end 152.476 90.536) (width 1) (layer "F.Cu") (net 22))
 (segment (start 148.59 78.486) (end 149.352 79.248) (width 1) (layer "F.Cu") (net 22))
 (segment (start 157.556 86.69) (end 156.464 85.598) (width 0.5) (layer "F.Cu") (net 25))
 (segment (start 156.464 85.598) (end 153.416 85.598) (width 0.5) (layer "F.Cu") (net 25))
 (segment (start 157.556 87.996) (end 157.556 86.69) (width 0.5) (layer "F.Cu") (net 25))
 (segment (start 153.416 85.598) (end 152.908 85.09) (width 0.5) (layer "F.Cu") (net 25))
 (segment (start 152.908 83.568) (end 153.128 83.568) (width 0.5) (layer "F.Cu") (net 25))
 (segment (start 152.908 83.568) (end 152.908 85.09) (width 0.5) (layer "F.Cu") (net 25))
 (segment (start 162.052 85.598) (end 162.636 86.182) (width 0.5) (layer "F.Cu") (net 26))
 (segment (start 157.556 83.642) (end 157.482 83.568) (width 0.5) (layer "F.Cu") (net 26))
 (segment (start 157.48 83.568) (end 158.208 83.568) (width 0.5) (layer "F.Cu") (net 26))
 (segment (start 157.988 85.598) (end 162.052 85.598) (width 0.5) (layer "F.Cu") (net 26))
 (segment (start 157.48 85.09) (end 157.988 85.598) (width 0.5) (layer "F.Cu") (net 26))
 (segment (start 157.48 83.568) (end 157.48 85.09) (width 0.5) (layer "F.Cu") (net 26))
 (segment (start 162.636 86.182) (end 162.636 87.996) (width 0.5) (layer "F.Cu") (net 26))
 (segment (start 79.572 71.897) (end 84.072 71.897) (width 1.5) (layer "F.Cu") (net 6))
 (segment (start 147.396 128.636) (end 147.396 131.176) (width 1) (layer "F.Cu") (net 1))
 (segment (start 142.316 131.176) (end 142.316 128.636) (width 1) (layer "F.Cu") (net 1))
 (segment (start 147.5955 135.382) (end 147.5955 131.3755) (width 0.5) (layer "F.Cu") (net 1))
 (segment (start 147.5955 131.3755) (end 147.396 131.176) (width 0.5) (layer "F.Cu") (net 1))
 (segment (start 141.222 133.86) (end 133.096 133.86) (width 1) (layer "B.Cu") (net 1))
 (segment (start 130.302 134.112) (end 132.844 134.112) (width 0.5) (layer "B.Cu") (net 1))
 (segment (start 129.794 131.8475) (end 129.794 133.604) (width 0.5) (layer "B.Cu") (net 1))
 (segment (start 142.316 131.176) (end 142.316 132.766) (width 1) (layer "B.Cu") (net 1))
 (segment (start 132.844 134.112) (end 133.096 133.86) (width 0.5) (layer "B.Cu") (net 1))
 (segment (start 129.794 133.604) (end 130.302 134.112) (width 0.5) (layer "B.Cu") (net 1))
 (segment (start 142.316 132.766) (end 141.222 133.86) (width 1) (layer "B.Cu") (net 1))
 (segment (start 145.5205 135.382) (end 143.258 135.382) (width 0.5) (layer "F.Cu") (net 2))
 (segment (start 145.5205 131.8405) (end 144.856 131.176) (width 0.5) (layer "F.Cu") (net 2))
 (segment (start 145.5205 135.382) (end 145.5205 131.8405) (width 0.5) (layer "F.Cu") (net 2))
 (segment (start 105.664 135.89) (end 106.426 136.652) (width 1) (layer "B.Cu") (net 2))
 (segment (start 105.664 134.1215) (end 105.664 135.89) (width 1) (layer "B.Cu") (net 2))
 (segment (start 144.856 135.458) (end 144.856 131.176) (width 1) (layer "B.Cu") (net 2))
 (segment (start 106.426 136.652) (end 142.494 136.652) (width 1) (layer "B.Cu") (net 2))
 (segment (start 143.662 136.652) (end 142.494 136.652) (width 1) (layer "B.Cu") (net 2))
 (segment (start 144.856 135.458) (end 143.662 136.652) (width 1) (layer "B.Cu") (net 2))
 (segment (start 129.616 87.996) (end 129.616 80.188) (width 1) (layer "F.Cu") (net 17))
 (segment (start 133.604 75.438) (end 135.128 75.438) (width 1) (layer "F.Cu") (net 17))
 (segment (start 133.096 78.526) (end 133.096 75.946) (width 1) (layer "F.Cu") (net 17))
 (segment (start 133.096 75.946) (end 133.604 75.438) (width 1) (layer "F.Cu") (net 17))
 (segment (start 131.278 78.526) (end 129.616 80.188) (width 1) (layer "F.Cu") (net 17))
 (segment (start 129.616 87.996) (end 129.616 90.536) (width 1) (layer "F.Cu") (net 17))
 (segment (start 135.636 72.015) (end 135.518 71.897) (width 1) (layer "F.Cu") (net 17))
 (segment (start 133.096 78.526) (end 131.278 78.526) (width 1) (layer "F.Cu") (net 17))
 (segment (start 135.636 74.93) (end 135.636 72.015) (width 1) (layer "F.Cu") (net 17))
 (segment (start 135.128 75.438) (end 135.636 74.93) (width 1) (layer "F.Cu") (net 17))
 (segment (start 129.616 93.906) (end 128.78 94.742) (width 1) (layer "B.Cu") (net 17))
 (segment (start 129.616 90.536) (end 129.616 93.906) (width 1) (layer "B.Cu") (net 17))
 (segment (start 163.83 93.218) (end 158.496 93.218) (width 0.5) (layer "F.Cu") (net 9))
 (segment (start 158.496 93.218) (end 157.556 92.278) (width 0.5) (layer "F.Cu") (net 9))
 (segment (start 164.846 84.074) (end 164.846 92.202) (width 0.5) (layer "F.Cu") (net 9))
 (segment (start 164.34 83.568) (end 164.846 84.074) (width 0.5) (layer "F.Cu") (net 9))
 (segment (start 162.054 83.568) (end 162.052 83.57) (width 0.5) (layer "F.Cu") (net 9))
 (segment (start 157.556 92.278) (end 157.556 90.536) (width 0.5) (layer "F.Cu") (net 9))
 (segment (start 164.846 92.202) (end 163.83 93.218) (width 0.5) (layer "F.Cu") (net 9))
 (segment (start 162.054 83.568) (end 164.34 83.568) (width 0.5) (layer "F.Cu") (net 9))
 (segment (start 137.236 135.304) (end 137.158 135.382) (width 1) (layer "F.Cu") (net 3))
 (segment (start 159.766 72.898) (end 159.766 78.232) (width 1) (layer "B.Cu") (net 10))
 (segment (start 160.274 78.74) (end 162.308 78.74) (width 1) (layer "B.Cu") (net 10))
 (segment (start 158.765 71.897) (end 159.766 72.898) (width 1) (layer "B.Cu") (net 10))
 (segment (start 157.018 71.897) (end 158.765 71.897) (width 1) (layer "B.Cu") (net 10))
 (segment (start 159.766 78.232) (end 160.274 78.74) (width 1) (layer "B.Cu") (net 10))
 (segment (start 100.076 129.286) (end 101.602 127.76) (width 1) (layer "B.Cu") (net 4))
 (segment (start 139.776 126.06) (end 139.192 125.476) (width 1) (layer "B.Cu") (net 4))
 (segment (start 139.776 128.636) (end 139.776 126.06) (width 1) (layer "B.Cu") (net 4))
 (segment (start 101.3555 134.1215) (end 100.076 132.842) (width 1) (layer "B.Cu") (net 4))
 (segment (start 133.096 127.76) (end 133.096 125.73) (width 1) (layer "B.Cu") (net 4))
 (segment (start 101.602 127.76) (end 133.096 127.76) (width 1) (layer "B.Cu") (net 4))
 (segment (start 138.938 125.222) (end 133.604 125.222) (width 1) (layer "B.Cu") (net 4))
 (segment (start 100.076 132.842) (end 100.076 129.286) (width 1) (layer "B.Cu") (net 4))
 (segment (start 139.192 125.476) (end 138.938 125.222) (width 1) (layer "B.Cu") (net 4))
 (segment (start 130.558 127.76) (end 133.096 127.76) (width 0.5) (layer "B.Cu") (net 4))
 (segment (start 133.096 125.73) (end 133.604 125.222) (width 1) (layer "B.Cu") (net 4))
 (segment (start 129.794 128.524) (end 130.558 127.76) (width 0.5) (layer "B.Cu") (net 4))
 (segment (start 129.794 129.7725) (end 129.794 128.524) (width 0.5) (layer "B.Cu") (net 4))
 (segment (start 103.124 134.1215) (end 101.3555 134.1215) (width 1) (layer "B.Cu") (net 4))
 (segment (start 62.572 71.897) (end 58.072 71.897) (width 1.5) (layer "F.Cu") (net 5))
 (segment (start 121.996 94.058) (end 122.68 94.742) (width 1) (layer "B.Cu") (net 12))
 (segment (start 121.996 90.536) (end 121.996 94.058) (width 1) (layer "B.Cu") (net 12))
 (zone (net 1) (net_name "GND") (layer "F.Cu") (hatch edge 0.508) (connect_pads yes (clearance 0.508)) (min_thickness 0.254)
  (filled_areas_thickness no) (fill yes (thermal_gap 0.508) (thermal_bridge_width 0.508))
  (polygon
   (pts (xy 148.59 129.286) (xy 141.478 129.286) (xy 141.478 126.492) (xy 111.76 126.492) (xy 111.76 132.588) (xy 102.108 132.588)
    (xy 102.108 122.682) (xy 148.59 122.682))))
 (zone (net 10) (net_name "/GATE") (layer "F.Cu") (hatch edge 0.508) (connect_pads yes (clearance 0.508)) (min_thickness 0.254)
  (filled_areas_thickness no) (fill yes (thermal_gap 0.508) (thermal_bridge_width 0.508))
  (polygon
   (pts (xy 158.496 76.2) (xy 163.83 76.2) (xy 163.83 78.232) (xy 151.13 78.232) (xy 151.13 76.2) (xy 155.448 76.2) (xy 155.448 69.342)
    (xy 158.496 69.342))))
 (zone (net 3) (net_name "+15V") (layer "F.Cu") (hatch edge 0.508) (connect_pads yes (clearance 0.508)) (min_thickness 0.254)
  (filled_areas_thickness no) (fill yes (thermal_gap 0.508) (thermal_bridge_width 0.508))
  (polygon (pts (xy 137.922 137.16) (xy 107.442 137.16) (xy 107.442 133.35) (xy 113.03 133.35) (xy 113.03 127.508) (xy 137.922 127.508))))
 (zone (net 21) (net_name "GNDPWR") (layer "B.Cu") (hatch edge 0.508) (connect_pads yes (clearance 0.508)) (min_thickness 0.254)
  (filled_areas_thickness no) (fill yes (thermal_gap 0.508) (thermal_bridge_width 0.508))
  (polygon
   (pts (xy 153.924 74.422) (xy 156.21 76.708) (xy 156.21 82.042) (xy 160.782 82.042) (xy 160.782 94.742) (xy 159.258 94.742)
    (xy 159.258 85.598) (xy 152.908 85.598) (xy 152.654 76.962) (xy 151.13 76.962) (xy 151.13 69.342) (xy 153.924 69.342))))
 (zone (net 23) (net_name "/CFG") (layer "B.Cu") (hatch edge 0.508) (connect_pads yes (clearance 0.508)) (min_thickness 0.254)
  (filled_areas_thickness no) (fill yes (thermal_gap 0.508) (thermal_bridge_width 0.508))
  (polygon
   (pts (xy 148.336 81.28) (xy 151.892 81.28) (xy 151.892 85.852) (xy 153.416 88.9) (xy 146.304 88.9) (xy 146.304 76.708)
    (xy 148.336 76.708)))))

